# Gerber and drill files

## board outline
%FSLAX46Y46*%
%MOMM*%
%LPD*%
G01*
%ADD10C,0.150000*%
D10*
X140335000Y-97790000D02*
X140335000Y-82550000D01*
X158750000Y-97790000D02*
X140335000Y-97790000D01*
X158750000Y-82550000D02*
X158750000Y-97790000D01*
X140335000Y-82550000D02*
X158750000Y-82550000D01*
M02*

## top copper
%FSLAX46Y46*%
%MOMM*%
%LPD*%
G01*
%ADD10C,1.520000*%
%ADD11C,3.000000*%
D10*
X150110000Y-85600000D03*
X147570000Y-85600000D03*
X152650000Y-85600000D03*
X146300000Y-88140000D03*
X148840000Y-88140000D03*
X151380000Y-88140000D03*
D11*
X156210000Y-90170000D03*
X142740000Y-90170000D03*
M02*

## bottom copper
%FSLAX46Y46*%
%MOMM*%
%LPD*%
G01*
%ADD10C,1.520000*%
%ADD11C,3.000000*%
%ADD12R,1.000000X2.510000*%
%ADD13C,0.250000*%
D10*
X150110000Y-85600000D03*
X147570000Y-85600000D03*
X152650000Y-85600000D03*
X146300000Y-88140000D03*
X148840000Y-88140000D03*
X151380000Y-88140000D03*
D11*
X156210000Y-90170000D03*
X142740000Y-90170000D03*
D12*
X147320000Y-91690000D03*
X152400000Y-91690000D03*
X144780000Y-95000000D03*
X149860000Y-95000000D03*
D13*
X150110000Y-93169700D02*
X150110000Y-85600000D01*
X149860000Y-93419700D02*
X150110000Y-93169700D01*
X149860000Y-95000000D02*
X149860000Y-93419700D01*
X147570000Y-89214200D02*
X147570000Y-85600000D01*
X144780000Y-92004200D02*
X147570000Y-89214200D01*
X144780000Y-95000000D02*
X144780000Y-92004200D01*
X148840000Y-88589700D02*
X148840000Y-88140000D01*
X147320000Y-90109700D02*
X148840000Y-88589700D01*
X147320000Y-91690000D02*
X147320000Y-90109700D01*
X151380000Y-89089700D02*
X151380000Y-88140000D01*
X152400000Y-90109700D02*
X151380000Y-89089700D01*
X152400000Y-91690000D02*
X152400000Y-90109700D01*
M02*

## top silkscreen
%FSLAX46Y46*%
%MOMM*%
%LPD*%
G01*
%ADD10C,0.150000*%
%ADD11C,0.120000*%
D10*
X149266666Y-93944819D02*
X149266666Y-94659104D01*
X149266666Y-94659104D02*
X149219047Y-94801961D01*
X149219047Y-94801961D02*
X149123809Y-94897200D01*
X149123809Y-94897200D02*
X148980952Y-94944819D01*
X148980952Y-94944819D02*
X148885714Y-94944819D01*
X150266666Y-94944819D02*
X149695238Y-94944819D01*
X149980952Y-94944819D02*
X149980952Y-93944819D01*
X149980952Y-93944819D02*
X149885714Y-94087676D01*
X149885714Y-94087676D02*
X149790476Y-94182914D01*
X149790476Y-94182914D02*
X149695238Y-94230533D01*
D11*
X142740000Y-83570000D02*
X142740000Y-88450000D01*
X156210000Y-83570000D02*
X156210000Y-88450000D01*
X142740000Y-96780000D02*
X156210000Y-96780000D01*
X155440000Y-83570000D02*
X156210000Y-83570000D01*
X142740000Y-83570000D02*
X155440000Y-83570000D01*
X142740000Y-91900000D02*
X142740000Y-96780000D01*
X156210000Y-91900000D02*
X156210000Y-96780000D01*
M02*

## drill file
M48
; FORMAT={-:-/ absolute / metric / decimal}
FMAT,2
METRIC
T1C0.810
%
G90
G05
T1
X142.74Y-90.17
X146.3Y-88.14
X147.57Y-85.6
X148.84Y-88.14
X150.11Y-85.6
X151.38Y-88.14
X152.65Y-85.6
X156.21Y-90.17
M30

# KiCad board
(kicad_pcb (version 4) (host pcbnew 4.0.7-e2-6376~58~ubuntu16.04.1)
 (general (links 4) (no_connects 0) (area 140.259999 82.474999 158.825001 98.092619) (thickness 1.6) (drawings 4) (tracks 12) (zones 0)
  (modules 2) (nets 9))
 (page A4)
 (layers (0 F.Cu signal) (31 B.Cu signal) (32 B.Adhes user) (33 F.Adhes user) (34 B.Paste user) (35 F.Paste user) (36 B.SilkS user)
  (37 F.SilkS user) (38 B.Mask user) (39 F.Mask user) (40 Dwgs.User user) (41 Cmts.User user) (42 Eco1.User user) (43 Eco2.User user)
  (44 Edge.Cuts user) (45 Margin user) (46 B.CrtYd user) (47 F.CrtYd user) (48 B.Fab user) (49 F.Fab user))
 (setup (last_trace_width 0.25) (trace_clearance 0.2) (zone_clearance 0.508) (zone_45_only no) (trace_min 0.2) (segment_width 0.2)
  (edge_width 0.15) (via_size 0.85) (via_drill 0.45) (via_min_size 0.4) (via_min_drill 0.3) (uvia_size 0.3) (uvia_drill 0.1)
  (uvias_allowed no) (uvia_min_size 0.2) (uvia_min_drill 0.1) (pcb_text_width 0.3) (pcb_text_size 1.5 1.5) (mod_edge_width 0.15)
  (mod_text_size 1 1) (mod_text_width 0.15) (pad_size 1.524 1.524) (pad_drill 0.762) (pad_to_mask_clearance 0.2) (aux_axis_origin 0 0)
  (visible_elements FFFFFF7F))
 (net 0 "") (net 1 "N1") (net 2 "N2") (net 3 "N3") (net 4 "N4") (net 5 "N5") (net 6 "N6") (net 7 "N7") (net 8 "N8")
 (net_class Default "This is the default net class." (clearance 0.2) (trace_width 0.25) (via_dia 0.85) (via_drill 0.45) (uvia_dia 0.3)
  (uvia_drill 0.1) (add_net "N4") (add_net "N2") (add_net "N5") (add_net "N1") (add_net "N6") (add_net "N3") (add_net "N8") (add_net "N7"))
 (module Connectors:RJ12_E (layer F.Cu) (at 146.3 88.14)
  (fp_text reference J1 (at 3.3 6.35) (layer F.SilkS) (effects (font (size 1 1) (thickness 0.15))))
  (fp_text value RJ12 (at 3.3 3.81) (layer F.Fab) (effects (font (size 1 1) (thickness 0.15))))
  (fp_line (start -3.56 -4.57) (end -3.56 0.31) (layer F.SilkS) (width 0.12))
  (fp_line (start 9.91 -4.57) (end 9.91 0.31) (layer F.SilkS) (width 0.12))
  (fp_line (start -3.56 8.64) (end 9.91 8.64) (layer F.SilkS) (width 0.12))
  (fp_line (start 9.14 -4.57) (end 9.91 -4.57) (layer F.SilkS) (width 0.12))
  (fp_line (start -3.56 -4.57) (end 9.14 -4.57) (layer F.SilkS) (width 0.12))
  (fp_line (start -3.56 3.76) (end -3.56 8.64) (layer F.SilkS) (width 0.12))
  (fp_line (start 9.91 3.76) (end 9.91 8.64) (layer F.SilkS) (width 0.12))
  (pad 4 thru_hole circle (at 3.81 -2.54) (size 1.52 1.52) (drill 0.81) (layers *.Cu *.Mask) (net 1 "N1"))
  (pad 2 thru_hole circle (at 1.27 -2.54) (size 1.52 1.52) (drill 0.81) (layers *.Cu *.Mask) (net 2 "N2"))
  (pad 6 thru_hole circle (at 6.35 -2.54) (size 1.52 1.52) (drill 0.81) (layers *.Cu *.Mask) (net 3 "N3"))
  (pad 1 thru_hole circle (at 0 0) (size 1.52 1.52) (drill 0.81) (layers *.Cu *.Mask) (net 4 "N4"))
  (pad 3 thru_hole circle (at 2.54 0) (size 1.52 1.52) (drill 0.81) (layers *.Cu *.Mask) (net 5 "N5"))
  (pad 5 thru_hole circle (at 5.08 0) (size 1.52 1.52) (drill 0.81) (layers *.Cu *.Mask) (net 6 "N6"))
  (pad 8 thru_hole circle (at 9.91 2.03) (size 3 3) (drill 0.81) (layers *.Cu *.Mask) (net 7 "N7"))
  (pad 7 thru_hole circle (at -3.56 2.03) (size 3 3) (drill 0.81) (layers *.Cu *.Mask) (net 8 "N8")))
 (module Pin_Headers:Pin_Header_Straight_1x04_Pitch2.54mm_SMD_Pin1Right (layer B.Cu) (at 148.59 93.345 270)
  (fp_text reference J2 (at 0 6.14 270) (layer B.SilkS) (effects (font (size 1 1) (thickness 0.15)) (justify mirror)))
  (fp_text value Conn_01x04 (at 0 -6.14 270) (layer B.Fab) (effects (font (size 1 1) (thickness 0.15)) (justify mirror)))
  (pad 2 smd rect (at -1.655 1.27 270) (size 2.51 1) (layers B.Cu B.Paste B.Mask) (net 5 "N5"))
  (pad 4 smd rect (at -1.655 -3.81 270) (size 2.51 1) (layers B.Cu B.Paste B.Mask) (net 6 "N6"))
  (pad 1 smd rect (at 1.655 3.81 270) (size 2.51 1) (layers B.Cu B.Paste B.Mask) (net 2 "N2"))
  (pad 3 smd rect (at 1.655 -1.27 270) (size 2.51 1) (layers B.Cu B.Paste B.Mask) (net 1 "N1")))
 (gr_line (start 140.335 97.79) (end 140.335 82.55) (layer Edge.Cuts) (width 0.15))
 (gr_line (start 158.75 97.79) (end 140.335 97.79) (layer Edge.Cuts) (width 0.15))
 (gr_line (start 158.75 82.55) (end 158.75 97.79) (layer Edge.Cuts) (width 0.15))
 (gr_line (start 140.335 82.55) (end 158.75 82.55) (layer Edge.Cuts) (width 0.15))
 (segment (start 150.11 93.1697) (end 150.11 85.6) (width 0.25) (layer B.Cu) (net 1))
 (segment (start 149.86 93.4197) (end 150.11 93.1697) (width 0.25) (layer B.Cu) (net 1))
 (segment (start 149.86 95) (end 149.86 93.4197) (width 0.25) (layer B.Cu) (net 1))
 (segment (start 147.57 89.2142) (end 147.57 85.6) (width 0.25) (layer B.Cu) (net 2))
 (segment (start 144.78 92.0042) (end 147.57 89.2142) (width 0.25) (layer B.Cu) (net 2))
 (segment (start 144.78 95) (end 144.78 92.0042) (width 0.25) (layer B.Cu) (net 2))
 (segment (start 148.84 88.5897) (end 148.84 88.14) (width 0.25) (layer B.Cu) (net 5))
 (segment (start 147.32 90.1097) (end 148.84 88.5897) (width 0.25) (layer B.Cu) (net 5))
 (segment (start 147.32 91.69) (end 147.32 90.1097) (width 0.25) (layer B.Cu) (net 5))
 (segment (start 151.38 89.0897) (end 151.38 88.14) (width 0.25) (layer B.Cu) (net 6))
 (segment (start 152.4 90.1097) (end 151.38 89.0897) (width 0.25) (layer B.Cu) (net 6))
 (segment (start 152.4 91.69) (end 152.4 90.1097) (width 0.25) (layer B.Cu) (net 6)))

